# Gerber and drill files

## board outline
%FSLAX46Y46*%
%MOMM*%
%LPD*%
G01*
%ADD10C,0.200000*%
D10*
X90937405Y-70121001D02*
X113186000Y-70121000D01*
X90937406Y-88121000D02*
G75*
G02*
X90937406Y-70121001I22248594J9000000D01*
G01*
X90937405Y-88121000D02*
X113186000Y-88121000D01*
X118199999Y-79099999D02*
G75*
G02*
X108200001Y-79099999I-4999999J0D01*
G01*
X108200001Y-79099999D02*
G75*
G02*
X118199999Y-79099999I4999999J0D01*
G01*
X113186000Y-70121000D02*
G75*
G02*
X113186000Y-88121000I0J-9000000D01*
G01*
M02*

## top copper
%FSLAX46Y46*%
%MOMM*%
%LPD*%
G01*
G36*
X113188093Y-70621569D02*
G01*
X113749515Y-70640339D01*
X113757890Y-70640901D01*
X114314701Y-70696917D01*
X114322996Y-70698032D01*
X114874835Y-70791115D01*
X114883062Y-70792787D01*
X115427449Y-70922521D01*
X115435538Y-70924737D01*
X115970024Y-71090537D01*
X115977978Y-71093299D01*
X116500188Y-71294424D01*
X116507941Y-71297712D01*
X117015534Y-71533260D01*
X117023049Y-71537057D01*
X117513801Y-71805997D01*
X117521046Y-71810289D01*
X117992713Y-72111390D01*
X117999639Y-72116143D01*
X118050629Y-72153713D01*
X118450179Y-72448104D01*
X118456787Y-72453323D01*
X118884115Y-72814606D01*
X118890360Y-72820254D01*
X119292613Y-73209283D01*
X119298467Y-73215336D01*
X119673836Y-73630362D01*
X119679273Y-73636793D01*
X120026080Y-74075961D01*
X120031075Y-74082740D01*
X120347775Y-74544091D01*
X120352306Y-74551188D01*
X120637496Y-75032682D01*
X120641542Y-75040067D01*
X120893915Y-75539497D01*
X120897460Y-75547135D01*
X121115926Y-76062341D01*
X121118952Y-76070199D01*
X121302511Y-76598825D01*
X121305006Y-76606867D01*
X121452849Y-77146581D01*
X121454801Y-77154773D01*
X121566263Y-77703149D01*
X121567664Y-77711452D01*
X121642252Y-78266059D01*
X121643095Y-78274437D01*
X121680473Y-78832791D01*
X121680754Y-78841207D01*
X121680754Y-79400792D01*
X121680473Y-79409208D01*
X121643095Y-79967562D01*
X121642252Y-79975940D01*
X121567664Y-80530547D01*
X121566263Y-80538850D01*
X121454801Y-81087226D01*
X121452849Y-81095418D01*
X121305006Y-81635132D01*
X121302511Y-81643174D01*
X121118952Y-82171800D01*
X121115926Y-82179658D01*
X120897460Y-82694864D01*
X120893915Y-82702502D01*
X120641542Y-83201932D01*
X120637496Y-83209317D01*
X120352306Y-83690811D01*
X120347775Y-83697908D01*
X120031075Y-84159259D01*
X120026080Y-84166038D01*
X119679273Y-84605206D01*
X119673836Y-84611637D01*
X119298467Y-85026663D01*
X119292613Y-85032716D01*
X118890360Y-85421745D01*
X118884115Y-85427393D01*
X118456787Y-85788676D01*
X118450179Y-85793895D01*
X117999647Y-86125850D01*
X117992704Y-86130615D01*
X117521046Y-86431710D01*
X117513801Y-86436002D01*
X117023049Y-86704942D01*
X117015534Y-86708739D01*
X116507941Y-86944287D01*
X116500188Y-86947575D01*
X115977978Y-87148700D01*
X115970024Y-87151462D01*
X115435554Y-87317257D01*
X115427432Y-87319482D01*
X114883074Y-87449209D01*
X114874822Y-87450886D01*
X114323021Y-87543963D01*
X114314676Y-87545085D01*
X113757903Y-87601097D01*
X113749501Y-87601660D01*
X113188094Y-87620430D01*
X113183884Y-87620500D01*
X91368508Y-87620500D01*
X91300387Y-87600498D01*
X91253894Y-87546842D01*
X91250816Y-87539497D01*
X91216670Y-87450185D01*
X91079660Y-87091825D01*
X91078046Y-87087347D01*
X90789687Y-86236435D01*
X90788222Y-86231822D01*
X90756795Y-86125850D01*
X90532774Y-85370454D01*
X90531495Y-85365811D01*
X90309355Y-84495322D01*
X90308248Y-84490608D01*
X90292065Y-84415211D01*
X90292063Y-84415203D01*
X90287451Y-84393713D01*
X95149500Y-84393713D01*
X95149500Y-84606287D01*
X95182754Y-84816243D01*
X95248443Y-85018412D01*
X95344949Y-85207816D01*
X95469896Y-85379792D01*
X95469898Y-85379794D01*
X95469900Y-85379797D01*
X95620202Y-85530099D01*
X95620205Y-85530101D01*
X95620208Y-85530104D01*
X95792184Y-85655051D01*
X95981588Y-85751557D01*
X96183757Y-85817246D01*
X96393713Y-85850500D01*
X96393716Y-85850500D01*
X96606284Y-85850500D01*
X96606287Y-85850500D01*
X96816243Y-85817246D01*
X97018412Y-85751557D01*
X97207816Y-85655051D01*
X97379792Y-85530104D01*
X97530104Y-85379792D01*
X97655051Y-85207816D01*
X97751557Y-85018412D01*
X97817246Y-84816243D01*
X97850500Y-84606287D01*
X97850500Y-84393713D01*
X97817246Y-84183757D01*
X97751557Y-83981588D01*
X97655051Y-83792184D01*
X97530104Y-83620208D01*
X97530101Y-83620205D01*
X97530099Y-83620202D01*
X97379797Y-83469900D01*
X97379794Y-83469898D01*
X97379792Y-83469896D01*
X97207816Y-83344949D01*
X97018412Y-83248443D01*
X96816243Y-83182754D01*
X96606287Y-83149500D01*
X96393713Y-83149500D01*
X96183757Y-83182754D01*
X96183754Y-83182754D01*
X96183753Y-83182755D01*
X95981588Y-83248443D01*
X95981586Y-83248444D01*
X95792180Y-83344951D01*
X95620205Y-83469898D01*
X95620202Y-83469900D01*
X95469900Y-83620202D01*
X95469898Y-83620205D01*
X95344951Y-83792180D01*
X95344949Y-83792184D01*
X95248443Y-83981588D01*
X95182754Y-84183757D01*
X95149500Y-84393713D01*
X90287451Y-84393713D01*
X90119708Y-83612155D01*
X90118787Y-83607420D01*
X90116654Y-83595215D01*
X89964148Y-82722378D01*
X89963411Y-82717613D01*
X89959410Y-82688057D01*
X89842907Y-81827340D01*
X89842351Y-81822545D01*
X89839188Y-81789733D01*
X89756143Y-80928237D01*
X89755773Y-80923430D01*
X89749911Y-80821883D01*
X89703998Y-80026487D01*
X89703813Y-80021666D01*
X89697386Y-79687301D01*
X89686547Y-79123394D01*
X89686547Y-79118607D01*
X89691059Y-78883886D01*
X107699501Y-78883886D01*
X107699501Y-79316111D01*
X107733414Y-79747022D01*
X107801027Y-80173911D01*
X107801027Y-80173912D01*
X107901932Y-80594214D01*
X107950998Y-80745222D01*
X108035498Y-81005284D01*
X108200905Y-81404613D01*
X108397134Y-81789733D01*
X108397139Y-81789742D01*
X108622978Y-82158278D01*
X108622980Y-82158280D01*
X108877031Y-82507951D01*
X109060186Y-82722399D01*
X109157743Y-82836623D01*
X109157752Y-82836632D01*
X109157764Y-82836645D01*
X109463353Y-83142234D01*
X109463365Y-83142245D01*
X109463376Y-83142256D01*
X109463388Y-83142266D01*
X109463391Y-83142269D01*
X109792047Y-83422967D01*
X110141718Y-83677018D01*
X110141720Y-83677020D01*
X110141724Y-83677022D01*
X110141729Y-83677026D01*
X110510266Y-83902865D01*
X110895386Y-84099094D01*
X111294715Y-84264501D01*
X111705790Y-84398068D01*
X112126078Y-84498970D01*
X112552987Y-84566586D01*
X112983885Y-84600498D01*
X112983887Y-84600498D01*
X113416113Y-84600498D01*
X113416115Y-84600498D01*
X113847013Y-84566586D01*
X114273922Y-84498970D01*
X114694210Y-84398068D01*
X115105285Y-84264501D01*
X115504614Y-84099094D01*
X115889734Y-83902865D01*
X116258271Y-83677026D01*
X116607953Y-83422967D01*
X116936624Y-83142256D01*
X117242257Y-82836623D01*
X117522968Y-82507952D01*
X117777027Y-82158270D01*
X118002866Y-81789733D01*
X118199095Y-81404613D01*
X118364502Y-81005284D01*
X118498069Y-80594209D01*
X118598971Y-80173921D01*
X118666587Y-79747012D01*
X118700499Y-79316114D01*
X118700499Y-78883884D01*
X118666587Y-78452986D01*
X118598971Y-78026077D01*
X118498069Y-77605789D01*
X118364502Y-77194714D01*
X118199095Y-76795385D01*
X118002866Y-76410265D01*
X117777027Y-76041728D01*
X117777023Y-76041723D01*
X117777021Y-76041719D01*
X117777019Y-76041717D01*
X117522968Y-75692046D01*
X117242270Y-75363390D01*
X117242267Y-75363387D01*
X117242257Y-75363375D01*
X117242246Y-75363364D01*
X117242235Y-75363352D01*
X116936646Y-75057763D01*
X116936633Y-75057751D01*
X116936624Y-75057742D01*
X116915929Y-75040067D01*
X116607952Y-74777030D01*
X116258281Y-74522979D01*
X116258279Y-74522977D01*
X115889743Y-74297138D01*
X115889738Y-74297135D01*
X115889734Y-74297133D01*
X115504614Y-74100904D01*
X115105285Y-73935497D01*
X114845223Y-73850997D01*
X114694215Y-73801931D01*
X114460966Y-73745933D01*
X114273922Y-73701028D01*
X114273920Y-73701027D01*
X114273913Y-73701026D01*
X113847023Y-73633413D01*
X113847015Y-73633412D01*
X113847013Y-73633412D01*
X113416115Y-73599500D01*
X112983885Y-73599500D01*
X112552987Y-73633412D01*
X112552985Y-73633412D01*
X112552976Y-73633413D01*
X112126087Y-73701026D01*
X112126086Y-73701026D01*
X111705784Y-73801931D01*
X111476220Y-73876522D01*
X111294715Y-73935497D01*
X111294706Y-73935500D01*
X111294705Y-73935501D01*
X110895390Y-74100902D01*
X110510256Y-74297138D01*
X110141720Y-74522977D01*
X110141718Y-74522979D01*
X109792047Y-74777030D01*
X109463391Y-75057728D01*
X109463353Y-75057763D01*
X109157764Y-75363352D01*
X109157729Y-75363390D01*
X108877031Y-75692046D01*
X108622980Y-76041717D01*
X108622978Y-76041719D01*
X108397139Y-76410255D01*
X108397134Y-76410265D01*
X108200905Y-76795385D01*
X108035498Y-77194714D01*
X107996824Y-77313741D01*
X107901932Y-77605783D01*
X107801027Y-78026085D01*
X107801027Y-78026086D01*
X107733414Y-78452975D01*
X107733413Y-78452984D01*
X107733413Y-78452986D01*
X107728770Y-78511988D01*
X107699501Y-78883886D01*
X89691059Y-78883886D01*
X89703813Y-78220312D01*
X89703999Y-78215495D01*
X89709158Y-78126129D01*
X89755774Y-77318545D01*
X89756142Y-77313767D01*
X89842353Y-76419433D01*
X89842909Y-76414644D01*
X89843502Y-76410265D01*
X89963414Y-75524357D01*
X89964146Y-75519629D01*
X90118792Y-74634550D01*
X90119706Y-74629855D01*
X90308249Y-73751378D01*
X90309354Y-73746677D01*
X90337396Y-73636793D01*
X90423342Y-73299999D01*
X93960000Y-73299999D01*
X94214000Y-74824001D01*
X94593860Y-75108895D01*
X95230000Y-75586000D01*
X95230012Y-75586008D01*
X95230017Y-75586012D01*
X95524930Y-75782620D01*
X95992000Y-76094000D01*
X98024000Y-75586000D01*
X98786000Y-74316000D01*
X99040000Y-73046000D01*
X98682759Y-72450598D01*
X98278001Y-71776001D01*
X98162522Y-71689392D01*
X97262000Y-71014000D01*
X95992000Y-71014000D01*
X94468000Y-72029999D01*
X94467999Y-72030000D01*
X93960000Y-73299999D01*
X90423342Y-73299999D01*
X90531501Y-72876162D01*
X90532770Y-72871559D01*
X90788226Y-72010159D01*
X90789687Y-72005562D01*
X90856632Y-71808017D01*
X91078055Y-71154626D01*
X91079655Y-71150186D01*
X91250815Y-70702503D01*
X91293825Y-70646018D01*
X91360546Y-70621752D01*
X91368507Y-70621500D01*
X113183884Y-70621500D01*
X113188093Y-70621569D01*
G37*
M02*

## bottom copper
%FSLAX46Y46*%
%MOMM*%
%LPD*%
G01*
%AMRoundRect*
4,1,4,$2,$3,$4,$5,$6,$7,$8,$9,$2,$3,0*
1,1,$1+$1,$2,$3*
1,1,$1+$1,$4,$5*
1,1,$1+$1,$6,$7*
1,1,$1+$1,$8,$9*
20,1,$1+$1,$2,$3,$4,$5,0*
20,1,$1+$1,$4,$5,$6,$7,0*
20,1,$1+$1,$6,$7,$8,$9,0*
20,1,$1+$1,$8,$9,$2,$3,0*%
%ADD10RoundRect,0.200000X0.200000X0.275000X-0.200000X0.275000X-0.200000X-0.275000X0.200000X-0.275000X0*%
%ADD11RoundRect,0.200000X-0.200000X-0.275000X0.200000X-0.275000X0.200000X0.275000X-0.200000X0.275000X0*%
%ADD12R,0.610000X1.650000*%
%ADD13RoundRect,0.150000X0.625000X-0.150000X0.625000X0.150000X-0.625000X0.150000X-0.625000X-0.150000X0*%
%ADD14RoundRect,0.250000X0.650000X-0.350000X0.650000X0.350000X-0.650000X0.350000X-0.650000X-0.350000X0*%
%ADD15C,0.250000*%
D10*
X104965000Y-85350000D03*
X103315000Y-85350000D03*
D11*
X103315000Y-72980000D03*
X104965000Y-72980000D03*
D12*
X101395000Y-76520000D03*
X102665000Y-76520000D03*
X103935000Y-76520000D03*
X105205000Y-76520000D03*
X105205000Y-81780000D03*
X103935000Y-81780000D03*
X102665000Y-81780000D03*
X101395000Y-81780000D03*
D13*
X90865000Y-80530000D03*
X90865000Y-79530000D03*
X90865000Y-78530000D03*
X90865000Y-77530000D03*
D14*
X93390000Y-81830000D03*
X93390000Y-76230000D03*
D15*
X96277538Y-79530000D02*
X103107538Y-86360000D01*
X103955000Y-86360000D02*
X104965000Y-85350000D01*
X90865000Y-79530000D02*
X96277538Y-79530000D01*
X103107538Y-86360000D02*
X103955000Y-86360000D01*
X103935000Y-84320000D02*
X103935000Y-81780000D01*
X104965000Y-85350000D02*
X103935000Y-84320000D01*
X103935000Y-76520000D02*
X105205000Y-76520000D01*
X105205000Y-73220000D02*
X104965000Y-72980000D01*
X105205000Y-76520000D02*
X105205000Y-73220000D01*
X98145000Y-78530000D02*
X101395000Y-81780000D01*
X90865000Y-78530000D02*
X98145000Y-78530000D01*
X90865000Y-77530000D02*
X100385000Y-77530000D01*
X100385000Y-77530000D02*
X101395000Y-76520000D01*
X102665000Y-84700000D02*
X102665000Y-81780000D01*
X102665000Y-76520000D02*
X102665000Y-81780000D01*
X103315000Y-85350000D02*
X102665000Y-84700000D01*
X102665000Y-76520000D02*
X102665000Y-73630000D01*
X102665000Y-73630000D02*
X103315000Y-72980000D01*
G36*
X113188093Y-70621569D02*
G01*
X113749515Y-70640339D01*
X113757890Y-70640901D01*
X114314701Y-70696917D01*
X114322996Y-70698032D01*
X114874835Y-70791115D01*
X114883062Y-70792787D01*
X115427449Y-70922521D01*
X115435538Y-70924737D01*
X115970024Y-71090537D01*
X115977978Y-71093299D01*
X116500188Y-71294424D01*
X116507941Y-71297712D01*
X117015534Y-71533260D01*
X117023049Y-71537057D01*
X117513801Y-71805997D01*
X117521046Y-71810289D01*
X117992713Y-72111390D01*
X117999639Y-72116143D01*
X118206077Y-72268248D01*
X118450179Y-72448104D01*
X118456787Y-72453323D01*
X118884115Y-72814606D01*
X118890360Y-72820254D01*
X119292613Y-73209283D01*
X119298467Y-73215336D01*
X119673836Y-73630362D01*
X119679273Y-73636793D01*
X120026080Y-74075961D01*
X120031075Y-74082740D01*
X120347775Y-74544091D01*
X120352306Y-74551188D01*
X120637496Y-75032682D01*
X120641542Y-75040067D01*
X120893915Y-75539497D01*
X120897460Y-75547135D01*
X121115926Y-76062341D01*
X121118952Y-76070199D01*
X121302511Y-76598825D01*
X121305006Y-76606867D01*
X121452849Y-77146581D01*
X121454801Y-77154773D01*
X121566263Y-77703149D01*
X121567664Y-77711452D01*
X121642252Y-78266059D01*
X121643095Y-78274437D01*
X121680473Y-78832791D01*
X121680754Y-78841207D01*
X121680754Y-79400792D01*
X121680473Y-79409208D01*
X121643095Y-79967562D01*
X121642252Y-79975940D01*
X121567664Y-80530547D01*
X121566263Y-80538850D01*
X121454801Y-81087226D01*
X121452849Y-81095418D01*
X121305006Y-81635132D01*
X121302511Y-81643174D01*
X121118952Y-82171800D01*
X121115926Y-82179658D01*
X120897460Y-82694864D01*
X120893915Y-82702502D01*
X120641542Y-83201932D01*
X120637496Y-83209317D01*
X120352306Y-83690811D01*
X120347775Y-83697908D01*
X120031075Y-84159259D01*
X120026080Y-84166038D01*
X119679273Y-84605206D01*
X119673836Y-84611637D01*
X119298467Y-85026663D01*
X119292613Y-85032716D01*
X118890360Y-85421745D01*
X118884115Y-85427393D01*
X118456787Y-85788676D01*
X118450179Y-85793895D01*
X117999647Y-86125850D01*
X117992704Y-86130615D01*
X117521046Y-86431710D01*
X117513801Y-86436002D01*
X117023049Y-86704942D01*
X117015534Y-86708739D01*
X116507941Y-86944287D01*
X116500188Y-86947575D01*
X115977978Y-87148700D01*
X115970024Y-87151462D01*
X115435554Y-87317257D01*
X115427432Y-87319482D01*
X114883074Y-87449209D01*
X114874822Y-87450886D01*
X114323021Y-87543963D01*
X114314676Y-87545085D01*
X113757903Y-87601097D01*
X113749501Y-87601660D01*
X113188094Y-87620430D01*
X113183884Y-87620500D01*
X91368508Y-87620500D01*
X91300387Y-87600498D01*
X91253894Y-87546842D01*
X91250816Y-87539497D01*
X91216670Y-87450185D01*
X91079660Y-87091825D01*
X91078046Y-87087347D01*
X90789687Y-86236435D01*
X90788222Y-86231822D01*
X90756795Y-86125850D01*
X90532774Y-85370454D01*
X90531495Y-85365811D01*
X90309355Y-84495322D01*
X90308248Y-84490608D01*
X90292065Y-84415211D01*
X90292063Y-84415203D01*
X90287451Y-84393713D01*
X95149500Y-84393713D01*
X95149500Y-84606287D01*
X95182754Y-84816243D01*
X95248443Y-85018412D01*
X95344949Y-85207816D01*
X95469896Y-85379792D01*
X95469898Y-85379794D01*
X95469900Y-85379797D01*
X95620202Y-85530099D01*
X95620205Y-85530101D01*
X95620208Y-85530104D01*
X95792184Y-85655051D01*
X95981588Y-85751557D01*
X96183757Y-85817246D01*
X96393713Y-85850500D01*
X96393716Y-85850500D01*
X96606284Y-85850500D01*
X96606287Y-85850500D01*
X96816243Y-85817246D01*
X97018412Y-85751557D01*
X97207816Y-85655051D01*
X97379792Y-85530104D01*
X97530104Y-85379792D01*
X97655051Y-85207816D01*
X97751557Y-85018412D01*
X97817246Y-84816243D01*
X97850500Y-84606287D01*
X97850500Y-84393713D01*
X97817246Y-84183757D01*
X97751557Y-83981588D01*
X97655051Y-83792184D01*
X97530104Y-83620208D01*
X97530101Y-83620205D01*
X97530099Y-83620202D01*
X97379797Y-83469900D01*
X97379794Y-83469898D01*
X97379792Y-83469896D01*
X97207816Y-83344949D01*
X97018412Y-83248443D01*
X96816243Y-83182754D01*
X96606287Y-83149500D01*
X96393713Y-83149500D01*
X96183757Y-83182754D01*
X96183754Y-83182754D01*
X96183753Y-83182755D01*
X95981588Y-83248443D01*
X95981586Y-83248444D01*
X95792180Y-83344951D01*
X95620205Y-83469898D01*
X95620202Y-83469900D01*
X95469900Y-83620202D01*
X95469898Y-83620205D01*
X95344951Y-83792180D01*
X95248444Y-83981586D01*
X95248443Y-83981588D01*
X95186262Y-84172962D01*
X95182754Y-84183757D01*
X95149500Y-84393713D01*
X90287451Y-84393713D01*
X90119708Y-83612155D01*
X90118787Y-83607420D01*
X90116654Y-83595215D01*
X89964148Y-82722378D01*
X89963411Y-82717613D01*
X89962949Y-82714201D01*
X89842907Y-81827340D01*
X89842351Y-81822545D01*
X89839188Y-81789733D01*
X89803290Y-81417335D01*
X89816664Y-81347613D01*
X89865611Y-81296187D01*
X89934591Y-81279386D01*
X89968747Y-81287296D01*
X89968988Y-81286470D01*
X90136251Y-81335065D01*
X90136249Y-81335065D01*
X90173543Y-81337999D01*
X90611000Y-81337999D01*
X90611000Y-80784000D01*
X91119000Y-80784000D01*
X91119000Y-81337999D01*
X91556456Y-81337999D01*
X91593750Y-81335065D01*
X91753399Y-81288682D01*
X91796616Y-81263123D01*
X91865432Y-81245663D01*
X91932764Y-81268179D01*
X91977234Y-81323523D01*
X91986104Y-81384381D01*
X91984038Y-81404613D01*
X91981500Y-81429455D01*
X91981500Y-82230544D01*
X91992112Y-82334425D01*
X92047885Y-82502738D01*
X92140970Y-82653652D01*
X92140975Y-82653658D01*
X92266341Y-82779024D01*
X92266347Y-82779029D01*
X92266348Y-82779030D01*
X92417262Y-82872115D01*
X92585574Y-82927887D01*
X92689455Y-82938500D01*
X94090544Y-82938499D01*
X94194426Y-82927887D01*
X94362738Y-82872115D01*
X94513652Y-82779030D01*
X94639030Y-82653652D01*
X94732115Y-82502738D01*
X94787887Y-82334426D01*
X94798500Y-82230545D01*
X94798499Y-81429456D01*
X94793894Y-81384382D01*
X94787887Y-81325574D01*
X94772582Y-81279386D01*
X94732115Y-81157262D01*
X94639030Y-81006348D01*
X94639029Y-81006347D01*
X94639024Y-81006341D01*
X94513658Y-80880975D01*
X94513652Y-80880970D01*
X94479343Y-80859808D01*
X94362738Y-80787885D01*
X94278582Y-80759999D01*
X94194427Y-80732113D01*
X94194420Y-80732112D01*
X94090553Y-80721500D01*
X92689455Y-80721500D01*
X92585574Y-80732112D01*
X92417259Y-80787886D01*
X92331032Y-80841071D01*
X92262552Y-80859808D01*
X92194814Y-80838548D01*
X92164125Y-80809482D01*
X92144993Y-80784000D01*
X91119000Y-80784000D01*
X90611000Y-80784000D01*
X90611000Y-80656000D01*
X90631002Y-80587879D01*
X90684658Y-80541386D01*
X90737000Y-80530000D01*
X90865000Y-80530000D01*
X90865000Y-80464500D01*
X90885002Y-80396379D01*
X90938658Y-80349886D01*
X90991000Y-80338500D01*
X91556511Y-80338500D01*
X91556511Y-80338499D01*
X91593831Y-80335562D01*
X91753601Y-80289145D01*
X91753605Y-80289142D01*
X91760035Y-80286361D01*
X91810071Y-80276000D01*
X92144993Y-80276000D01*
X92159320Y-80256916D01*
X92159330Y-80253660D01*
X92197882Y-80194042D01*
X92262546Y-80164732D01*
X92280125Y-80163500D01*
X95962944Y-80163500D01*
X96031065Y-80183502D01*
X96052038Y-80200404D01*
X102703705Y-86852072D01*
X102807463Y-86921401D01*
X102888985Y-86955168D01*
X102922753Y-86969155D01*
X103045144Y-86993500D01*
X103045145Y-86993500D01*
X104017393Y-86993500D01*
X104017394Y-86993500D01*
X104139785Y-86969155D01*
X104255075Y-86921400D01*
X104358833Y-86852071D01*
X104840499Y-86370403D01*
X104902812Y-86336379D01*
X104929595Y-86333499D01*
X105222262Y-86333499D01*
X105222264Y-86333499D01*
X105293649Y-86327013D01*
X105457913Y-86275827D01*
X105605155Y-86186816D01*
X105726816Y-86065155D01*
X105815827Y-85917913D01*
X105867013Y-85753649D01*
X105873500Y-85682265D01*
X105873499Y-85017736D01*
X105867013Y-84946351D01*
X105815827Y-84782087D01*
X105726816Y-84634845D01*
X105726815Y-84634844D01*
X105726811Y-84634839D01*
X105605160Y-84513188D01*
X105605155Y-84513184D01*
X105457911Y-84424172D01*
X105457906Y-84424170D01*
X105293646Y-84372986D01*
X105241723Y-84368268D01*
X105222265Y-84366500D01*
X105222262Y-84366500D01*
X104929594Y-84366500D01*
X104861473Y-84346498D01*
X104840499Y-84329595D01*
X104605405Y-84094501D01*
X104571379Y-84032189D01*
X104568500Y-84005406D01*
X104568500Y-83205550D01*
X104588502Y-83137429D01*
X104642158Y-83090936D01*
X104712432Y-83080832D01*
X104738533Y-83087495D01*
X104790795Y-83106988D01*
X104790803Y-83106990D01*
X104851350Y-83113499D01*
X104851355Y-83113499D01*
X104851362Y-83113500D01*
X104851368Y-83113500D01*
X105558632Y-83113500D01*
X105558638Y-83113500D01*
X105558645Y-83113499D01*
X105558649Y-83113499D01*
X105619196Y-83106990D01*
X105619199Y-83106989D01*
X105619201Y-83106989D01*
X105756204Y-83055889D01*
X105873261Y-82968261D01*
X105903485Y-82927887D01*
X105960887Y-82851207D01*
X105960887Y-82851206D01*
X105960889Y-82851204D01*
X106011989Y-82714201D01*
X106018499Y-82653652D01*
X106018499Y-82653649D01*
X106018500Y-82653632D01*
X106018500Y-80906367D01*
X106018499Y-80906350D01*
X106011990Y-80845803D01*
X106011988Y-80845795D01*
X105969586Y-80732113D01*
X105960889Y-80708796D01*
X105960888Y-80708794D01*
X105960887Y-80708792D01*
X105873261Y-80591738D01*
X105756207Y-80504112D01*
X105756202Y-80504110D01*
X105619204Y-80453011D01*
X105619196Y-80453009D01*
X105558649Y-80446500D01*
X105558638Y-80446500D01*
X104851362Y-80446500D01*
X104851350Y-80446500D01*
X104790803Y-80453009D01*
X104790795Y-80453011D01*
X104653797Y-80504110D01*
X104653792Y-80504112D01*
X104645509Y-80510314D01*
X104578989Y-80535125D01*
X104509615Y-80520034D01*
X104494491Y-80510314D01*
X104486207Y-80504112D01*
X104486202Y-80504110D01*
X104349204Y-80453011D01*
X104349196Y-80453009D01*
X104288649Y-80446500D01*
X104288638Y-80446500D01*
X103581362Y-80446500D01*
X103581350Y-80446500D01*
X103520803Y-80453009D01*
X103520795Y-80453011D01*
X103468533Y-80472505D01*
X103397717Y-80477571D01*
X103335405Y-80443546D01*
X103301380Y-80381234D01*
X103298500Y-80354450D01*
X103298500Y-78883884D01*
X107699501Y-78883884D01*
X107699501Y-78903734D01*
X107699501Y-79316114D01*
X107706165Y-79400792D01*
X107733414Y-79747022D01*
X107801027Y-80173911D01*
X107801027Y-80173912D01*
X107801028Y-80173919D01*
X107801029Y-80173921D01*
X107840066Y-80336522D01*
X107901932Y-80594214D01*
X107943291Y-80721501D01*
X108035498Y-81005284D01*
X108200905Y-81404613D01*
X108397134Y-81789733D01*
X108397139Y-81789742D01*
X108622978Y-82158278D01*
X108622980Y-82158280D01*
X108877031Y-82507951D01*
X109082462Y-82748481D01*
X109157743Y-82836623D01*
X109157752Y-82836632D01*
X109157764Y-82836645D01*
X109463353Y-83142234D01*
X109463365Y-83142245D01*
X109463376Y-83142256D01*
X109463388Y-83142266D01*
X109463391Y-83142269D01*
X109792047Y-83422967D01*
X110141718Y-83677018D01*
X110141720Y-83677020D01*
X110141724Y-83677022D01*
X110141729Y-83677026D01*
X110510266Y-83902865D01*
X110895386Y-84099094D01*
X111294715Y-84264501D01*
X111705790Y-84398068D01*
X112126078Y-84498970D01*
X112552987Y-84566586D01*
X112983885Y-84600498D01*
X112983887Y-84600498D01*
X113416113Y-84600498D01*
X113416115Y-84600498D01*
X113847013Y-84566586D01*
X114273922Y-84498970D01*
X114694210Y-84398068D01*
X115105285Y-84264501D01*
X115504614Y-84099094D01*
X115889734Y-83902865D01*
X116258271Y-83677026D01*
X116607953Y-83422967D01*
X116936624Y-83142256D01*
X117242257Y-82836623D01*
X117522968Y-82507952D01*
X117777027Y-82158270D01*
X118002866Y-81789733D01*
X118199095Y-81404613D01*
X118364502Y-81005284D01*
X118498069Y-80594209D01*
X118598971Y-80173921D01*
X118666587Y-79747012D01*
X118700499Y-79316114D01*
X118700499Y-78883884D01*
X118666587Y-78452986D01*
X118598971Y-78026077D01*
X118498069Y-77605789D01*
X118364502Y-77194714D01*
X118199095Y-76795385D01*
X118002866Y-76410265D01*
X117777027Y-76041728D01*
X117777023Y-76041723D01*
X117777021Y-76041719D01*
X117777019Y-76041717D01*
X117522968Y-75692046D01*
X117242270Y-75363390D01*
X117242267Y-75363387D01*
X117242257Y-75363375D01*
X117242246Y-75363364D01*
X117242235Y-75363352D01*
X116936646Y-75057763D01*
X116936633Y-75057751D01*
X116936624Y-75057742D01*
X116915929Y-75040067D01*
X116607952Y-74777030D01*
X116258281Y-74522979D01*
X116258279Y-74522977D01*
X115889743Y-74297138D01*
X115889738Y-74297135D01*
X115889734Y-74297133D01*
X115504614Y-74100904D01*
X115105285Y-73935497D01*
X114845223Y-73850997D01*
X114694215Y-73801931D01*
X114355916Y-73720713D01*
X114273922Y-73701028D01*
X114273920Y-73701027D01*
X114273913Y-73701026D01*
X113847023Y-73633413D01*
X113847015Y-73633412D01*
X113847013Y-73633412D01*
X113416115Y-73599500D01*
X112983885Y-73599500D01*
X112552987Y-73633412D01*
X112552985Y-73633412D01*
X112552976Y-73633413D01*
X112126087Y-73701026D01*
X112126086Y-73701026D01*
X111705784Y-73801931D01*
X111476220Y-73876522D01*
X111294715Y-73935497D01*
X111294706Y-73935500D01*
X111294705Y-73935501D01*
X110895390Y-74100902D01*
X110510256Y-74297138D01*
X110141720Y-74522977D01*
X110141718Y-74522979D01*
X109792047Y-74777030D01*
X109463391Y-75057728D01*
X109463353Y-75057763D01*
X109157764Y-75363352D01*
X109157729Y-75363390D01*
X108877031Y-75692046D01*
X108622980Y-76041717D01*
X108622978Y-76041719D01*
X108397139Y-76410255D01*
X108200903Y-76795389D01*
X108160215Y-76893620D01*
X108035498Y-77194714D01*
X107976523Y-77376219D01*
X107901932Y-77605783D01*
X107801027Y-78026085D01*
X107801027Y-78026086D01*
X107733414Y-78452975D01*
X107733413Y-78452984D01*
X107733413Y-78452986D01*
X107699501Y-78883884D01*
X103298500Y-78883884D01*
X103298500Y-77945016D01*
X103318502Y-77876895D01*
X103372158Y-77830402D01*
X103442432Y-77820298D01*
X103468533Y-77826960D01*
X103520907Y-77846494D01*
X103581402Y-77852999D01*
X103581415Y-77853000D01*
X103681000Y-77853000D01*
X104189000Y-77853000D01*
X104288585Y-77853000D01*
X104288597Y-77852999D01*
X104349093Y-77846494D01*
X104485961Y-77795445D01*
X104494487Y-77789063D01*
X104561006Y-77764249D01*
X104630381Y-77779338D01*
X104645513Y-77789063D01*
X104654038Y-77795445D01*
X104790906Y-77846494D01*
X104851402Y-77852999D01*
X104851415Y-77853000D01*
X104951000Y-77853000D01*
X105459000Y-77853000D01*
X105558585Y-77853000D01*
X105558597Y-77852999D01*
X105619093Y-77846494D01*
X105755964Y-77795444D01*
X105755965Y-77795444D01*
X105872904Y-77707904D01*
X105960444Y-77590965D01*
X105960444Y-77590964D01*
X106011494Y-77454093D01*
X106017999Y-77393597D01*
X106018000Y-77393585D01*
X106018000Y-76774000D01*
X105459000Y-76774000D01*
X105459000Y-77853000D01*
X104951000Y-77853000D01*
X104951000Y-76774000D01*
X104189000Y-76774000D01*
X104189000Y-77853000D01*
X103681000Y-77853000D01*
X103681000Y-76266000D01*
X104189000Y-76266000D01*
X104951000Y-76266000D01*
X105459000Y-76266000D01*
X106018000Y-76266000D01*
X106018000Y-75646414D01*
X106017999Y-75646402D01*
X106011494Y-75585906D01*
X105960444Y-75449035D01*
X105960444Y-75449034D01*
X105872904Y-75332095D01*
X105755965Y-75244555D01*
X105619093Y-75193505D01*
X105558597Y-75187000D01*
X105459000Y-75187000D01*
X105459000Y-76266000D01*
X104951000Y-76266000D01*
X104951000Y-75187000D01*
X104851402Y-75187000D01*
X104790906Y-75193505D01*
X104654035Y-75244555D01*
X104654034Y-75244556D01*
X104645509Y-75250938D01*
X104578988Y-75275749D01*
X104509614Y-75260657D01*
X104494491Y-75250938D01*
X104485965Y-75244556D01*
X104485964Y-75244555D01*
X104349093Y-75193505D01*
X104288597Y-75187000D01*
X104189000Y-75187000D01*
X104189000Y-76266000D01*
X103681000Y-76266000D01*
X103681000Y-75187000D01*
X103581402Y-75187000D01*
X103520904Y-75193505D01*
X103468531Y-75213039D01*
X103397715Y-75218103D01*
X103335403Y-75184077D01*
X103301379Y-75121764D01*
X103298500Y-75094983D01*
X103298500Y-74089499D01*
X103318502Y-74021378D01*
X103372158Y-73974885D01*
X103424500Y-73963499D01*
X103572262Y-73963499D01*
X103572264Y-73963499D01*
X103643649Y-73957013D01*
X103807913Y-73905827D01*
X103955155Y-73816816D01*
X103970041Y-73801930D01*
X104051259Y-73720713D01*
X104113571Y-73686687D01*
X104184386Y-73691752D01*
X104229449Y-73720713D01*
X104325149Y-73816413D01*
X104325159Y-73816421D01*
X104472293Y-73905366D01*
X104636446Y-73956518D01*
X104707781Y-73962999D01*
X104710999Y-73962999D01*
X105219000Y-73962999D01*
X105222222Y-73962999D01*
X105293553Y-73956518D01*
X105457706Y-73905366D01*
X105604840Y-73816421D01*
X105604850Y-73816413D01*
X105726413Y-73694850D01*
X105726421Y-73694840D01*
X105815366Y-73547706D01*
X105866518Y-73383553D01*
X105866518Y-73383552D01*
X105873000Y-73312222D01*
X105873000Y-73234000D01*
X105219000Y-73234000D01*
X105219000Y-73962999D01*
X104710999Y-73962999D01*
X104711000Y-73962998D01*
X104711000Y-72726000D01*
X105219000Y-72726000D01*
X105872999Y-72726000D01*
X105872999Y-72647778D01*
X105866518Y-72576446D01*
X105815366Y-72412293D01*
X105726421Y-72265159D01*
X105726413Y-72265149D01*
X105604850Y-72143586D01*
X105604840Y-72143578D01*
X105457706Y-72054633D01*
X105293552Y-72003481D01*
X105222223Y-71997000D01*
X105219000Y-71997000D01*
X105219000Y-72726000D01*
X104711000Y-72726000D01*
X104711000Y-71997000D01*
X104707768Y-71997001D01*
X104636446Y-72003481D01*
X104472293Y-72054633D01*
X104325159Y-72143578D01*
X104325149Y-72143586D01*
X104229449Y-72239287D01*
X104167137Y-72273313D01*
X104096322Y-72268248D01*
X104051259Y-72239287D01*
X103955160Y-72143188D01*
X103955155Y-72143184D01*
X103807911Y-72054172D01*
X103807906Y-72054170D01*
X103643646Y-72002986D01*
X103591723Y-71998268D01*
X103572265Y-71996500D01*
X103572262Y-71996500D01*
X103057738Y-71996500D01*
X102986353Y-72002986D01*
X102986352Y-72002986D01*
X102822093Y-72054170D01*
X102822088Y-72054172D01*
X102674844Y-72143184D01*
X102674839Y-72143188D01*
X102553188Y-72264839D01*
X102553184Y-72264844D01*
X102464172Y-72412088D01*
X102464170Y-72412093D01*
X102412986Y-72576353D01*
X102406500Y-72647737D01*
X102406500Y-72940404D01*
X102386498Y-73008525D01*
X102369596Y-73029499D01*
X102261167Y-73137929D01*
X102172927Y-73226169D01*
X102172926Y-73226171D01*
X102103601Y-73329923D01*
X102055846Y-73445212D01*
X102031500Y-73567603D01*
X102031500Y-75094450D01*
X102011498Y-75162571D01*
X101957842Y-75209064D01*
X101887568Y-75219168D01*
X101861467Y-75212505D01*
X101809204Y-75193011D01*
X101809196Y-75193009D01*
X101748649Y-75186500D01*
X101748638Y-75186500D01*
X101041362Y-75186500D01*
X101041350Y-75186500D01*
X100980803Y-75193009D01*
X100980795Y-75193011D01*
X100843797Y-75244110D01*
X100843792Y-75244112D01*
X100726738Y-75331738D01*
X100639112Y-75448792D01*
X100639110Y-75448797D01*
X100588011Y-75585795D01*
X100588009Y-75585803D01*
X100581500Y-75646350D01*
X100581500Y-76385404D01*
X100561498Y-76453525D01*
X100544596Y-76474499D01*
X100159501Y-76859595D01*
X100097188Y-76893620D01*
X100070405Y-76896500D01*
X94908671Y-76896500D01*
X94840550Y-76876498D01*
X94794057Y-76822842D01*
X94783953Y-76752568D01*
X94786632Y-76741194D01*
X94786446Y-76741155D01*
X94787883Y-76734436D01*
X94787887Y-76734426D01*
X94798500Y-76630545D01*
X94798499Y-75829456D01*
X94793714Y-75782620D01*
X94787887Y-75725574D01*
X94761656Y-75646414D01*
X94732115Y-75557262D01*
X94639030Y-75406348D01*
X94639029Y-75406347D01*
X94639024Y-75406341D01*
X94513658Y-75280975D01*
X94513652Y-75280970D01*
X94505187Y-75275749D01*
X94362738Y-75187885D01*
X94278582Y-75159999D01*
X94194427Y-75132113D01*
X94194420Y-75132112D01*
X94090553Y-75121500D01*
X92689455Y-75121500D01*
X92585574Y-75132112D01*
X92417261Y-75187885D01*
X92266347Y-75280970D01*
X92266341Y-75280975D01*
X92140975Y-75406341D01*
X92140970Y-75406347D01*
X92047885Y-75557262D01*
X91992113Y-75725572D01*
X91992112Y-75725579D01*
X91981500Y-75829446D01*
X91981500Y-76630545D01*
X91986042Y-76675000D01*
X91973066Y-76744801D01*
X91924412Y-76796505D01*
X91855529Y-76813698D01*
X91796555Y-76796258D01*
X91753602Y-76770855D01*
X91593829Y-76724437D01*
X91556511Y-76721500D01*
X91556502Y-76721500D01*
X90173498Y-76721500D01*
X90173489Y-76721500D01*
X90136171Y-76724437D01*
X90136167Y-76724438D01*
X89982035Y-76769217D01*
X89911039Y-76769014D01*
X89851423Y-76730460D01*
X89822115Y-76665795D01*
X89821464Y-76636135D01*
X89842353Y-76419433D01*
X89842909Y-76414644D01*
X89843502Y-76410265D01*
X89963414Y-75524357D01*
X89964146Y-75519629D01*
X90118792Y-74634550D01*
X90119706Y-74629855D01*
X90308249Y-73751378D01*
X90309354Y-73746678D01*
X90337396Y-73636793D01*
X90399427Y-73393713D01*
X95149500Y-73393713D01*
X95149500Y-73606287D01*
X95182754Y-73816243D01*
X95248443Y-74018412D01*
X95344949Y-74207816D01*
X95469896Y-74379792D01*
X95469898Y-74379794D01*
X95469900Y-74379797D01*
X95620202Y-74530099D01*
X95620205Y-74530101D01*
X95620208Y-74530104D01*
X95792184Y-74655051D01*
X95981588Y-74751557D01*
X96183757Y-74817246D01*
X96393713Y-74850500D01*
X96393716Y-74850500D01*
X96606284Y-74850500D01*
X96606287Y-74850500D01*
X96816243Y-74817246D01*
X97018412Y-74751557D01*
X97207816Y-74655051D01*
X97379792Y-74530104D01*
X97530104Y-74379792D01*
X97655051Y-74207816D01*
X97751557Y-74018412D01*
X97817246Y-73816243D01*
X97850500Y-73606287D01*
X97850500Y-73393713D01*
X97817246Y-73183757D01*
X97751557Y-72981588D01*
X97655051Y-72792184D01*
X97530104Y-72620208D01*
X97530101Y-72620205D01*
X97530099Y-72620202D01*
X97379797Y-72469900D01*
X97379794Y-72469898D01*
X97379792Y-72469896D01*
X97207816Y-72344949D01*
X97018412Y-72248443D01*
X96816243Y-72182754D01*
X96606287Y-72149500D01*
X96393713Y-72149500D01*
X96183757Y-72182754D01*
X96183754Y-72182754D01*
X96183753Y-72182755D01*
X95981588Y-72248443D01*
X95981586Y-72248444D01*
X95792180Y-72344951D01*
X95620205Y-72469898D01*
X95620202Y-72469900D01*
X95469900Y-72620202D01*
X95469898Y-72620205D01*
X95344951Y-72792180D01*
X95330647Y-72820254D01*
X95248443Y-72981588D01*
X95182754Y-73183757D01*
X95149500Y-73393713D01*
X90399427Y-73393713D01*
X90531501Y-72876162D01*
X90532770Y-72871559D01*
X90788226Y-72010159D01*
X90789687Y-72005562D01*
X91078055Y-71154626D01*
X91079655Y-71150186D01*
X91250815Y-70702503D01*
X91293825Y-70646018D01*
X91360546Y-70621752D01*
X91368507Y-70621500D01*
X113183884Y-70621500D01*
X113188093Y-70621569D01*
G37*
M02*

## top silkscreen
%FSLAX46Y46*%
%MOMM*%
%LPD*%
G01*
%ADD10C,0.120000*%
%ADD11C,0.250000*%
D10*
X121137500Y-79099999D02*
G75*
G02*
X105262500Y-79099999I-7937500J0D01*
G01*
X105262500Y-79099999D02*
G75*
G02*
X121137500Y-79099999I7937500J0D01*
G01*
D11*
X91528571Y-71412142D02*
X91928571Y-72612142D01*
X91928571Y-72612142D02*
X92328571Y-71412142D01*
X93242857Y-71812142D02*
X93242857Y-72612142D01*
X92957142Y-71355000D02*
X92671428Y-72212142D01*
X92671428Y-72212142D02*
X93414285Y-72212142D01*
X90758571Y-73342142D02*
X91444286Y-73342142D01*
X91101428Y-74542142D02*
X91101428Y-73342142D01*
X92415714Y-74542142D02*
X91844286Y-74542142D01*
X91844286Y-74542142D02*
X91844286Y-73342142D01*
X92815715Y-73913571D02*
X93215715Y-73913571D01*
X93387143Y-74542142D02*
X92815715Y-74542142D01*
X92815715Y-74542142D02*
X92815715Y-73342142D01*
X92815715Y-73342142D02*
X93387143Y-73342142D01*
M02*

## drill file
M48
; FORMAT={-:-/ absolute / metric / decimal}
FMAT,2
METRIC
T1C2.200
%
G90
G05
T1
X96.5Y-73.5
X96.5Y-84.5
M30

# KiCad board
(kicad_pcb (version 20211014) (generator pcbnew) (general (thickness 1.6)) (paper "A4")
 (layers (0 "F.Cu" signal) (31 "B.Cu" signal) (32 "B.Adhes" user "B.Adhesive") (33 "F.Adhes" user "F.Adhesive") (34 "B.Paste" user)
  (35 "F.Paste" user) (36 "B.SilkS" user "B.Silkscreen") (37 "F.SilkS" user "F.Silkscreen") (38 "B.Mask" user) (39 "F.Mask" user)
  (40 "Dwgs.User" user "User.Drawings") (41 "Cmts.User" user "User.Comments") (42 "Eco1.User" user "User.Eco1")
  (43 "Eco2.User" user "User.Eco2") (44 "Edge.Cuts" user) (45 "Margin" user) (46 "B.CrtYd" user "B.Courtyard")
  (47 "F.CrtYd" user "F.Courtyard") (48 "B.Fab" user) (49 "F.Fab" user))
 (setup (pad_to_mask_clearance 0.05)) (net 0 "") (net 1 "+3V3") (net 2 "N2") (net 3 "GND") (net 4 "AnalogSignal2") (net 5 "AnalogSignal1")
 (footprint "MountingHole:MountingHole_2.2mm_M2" (layer "F.Cu") (at 96.5 84.5)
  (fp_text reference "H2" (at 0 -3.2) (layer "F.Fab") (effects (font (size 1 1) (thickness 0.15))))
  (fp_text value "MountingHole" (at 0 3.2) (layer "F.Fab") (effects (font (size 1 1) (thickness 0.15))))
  (pad "" np_thru_hole circle locked (at 0 0) (size 2.2 2.2) (drill 2.2) (layers *.Cu *.Mask)))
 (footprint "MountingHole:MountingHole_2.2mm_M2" (layer "F.Cu") (at 96.5 73.5)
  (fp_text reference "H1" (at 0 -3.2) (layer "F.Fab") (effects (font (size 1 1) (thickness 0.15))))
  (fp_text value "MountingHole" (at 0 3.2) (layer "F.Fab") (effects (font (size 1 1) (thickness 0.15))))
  (pad "" np_thru_hole circle locked (at 0 0) (size 2.2 2.2) (drill 2.2) (layers *.Cu *.Mask)))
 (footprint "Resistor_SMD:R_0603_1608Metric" (layer "B.Cu") (at 104.14 85.35 180)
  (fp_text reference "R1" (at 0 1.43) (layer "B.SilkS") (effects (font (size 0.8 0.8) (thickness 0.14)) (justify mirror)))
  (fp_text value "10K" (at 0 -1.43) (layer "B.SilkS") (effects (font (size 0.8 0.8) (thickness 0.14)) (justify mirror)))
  (pad "1" smd roundrect locked (at -0.825 0 180) (size 0.8 0.95) (layers "B.Cu" "B.Paste" "B.Mask") (roundrect_rratio 0.25) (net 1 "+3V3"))
  (pad "2" smd roundrect locked (at 0.825 0 180) (size 0.8 0.95) (layers "B.Cu" "B.Paste" "B.Mask") (roundrect_rratio 0.25) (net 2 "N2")))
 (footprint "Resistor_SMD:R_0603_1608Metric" (layer "B.Cu") (at 104.14 72.98)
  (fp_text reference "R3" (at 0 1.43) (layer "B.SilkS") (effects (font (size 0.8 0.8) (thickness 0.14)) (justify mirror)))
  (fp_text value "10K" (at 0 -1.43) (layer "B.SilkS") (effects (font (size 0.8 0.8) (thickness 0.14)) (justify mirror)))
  (pad "1" smd roundrect locked (at -0.825 0) (size 0.8 0.95) (layers "B.Cu" "B.Paste" "B.Mask") (roundrect_rratio 0.25) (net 2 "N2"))
  (pad "2" smd roundrect locked (at 0.825 0) (size 0.8 0.95) (layers "B.Cu" "B.Paste" "B.Mask") (roundrect_rratio 0.25) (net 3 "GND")))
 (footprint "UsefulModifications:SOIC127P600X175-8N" (layer "B.Cu") (at 103.3 79.15 -90)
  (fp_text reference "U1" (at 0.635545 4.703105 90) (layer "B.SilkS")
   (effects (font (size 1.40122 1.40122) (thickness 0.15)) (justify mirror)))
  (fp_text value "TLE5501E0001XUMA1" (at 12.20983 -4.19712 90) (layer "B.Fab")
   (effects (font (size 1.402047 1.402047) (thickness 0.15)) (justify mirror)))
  (pad "1" smd rect locked (at -2.63 1.905 270) (size 1.65 0.61) (layers "B.Cu" "B.Paste" "B.Mask") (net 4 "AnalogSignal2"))
  (pad "2" smd rect locked (at -2.63 0.635 270) (size 1.65 0.61) (layers "B.Cu" "B.Paste" "B.Mask") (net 2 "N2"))
  (pad "3" smd rect locked (at -2.63 -0.635 270) (size 1.65 0.61) (layers "B.Cu" "B.Paste" "B.Mask") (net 3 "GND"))
  (pad "4" smd rect locked (at -2.63 -1.905 270) (size 1.65 0.61) (layers "B.Cu" "B.Paste" "B.Mask") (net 3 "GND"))
  (pad "5" smd rect locked (at 2.63 -1.905 270) (size 1.65 0.61) (layers "B.Cu" "B.Paste" "B.Mask"))
  (pad "6" smd rect locked (at 2.63 -0.635 270) (size 1.65 0.61) (layers "B.Cu" "B.Paste" "B.Mask") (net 1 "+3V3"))
  (pad "7" smd rect locked (at 2.63 0.635 270) (size 1.65 0.61) (layers "B.Cu" "B.Paste" "B.Mask") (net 2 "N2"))
  (pad "8" smd rect locked (at 2.63 1.905 270) (size 1.65 0.61) (layers "B.Cu" "B.Paste" "B.Mask") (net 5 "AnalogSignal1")))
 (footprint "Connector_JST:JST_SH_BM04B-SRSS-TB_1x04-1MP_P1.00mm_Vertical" (layer "B.Cu") (at 92.19 79.03 90)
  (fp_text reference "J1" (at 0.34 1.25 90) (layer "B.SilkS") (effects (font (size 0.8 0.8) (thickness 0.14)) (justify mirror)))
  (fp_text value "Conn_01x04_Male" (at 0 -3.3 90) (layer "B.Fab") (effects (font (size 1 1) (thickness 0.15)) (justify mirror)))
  (pad "1" smd roundrect locked (at -1.5 -1.325 90) (size 0.6 1.55) (layers "B.Cu" "B.Paste" "B.Mask") (roundrect_rratio 0.25) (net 3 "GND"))
  (pad "2" smd roundrect locked (at -0.5 -1.325 90) (size 0.6 1.55) (layers "B.Cu" "B.Paste" "B.Mask") (roundrect_rratio 0.25)
   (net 1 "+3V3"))
  (pad "3" smd roundrect locked (at 0.5 -1.325 90) (size 0.6 1.55) (layers "B.Cu" "B.Paste" "B.Mask") (roundrect_rratio 0.25)
   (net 5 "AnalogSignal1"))
  (pad "4" smd roundrect locked (at 1.5 -1.325 90) (size 0.6 1.55) (layers "B.Cu" "B.Paste" "B.Mask") (roundrect_rratio 0.25)
   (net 4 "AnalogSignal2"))
  (pad "MP" smd roundrect locked (at -2.8 1.2 90) (size 1.2 1.8) (layers "B.Cu" "B.Paste" "B.Mask") (roundrect_rratio 0.2083333333))
  (pad "MP" smd roundrect locked (at 2.8 1.2 90) (size 1.2 1.8) (layers "B.Cu" "B.Paste" "B.Mask") (roundrect_rratio 0.2083333333)))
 (gr_circle (center 113.2 79.099999) (end 121.1375 79.099999) (layer "F.SilkS") (width 0.12) (fill none))
 (gr_line (start 90.937405 70.121001) (end 113.186 70.121) (layer "Edge.Cuts") (width 0.2))
 (gr_arc (start 90.937406 88.121) (mid 89.186001 79.121001) (end 90.937405 70.121001) (layer "Edge.Cuts") (width 0.2))
 (gr_line (start 90.937405 88.121) (end 113.186 88.121) (layer "Edge.Cuts") (width 0.2))
 (gr_circle (center 113.2 79.099999) (end 118.199999 79.099999) (layer "Edge.Cuts") (width 0.2) (fill none))
 (gr_arc (start 113.186 70.121) (mid 122.186 79.121) (end 113.186 88.121) (layer "Edge.Cuts") (width 0.2))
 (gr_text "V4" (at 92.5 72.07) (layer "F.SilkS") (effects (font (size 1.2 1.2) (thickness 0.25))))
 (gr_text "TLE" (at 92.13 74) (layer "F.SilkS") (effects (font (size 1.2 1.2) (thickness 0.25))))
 (segment (start 96.277538 79.53) (end 103.107538 86.36) (width 0.25) (layer "B.Cu") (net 1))
 (segment (start 103.955 86.36) (end 104.965 85.35) (width 0.25) (layer "B.Cu") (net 1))
 (segment (start 90.865 79.53) (end 96.277538 79.53) (width 0.25) (layer "B.Cu") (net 1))
 (segment (start 103.107538 86.36) (end 103.955 86.36) (width 0.25) (layer "B.Cu") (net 1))
 (segment (start 103.935 84.32) (end 103.935 81.78) (width 0.25) (layer "B.Cu") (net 1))
 (segment (start 104.965 85.35) (end 103.935 84.32) (width 0.25) (layer "B.Cu") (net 1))
 (segment (start 103.935 76.52) (end 105.205 76.52) (width 0.25) (layer "B.Cu") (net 3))
 (segment (start 105.205 73.22) (end 104.965 72.98) (width 0.25) (layer "B.Cu") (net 3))
 (segment (start 105.205 76.52) (end 105.205 73.22) (width 0.25) (layer "B.Cu") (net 3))
 (segment (start 98.145 78.53) (end 101.395 81.78) (width 0.25) (layer "B.Cu") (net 5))
 (segment (start 90.865 78.53) (end 98.145 78.53) (width 0.25) (layer "B.Cu") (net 5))
 (segment (start 90.865 77.53) (end 100.385 77.53) (width 0.25) (layer "B.Cu") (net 4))
 (segment (start 100.385 77.53) (end 101.395 76.52) (width 0.25) (layer "B.Cu") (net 4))
 (segment (start 102.665 84.7) (end 102.665 81.78) (width 0.25) (layer "B.Cu") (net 2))
 (segment (start 102.665 76.52) (end 102.665 81.78) (width 0.25) (layer "B.Cu") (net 2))
 (segment (start 103.315 85.35) (end 102.665 84.7) (width 0.25) (layer "B.Cu") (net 2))
 (segment (start 102.665 76.52) (end 102.665 73.63) (width 0.25) (layer "B.Cu") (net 2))
 (segment (start 102.665 73.63) (end 103.315 72.98) (width 0.25) (layer "B.Cu") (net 2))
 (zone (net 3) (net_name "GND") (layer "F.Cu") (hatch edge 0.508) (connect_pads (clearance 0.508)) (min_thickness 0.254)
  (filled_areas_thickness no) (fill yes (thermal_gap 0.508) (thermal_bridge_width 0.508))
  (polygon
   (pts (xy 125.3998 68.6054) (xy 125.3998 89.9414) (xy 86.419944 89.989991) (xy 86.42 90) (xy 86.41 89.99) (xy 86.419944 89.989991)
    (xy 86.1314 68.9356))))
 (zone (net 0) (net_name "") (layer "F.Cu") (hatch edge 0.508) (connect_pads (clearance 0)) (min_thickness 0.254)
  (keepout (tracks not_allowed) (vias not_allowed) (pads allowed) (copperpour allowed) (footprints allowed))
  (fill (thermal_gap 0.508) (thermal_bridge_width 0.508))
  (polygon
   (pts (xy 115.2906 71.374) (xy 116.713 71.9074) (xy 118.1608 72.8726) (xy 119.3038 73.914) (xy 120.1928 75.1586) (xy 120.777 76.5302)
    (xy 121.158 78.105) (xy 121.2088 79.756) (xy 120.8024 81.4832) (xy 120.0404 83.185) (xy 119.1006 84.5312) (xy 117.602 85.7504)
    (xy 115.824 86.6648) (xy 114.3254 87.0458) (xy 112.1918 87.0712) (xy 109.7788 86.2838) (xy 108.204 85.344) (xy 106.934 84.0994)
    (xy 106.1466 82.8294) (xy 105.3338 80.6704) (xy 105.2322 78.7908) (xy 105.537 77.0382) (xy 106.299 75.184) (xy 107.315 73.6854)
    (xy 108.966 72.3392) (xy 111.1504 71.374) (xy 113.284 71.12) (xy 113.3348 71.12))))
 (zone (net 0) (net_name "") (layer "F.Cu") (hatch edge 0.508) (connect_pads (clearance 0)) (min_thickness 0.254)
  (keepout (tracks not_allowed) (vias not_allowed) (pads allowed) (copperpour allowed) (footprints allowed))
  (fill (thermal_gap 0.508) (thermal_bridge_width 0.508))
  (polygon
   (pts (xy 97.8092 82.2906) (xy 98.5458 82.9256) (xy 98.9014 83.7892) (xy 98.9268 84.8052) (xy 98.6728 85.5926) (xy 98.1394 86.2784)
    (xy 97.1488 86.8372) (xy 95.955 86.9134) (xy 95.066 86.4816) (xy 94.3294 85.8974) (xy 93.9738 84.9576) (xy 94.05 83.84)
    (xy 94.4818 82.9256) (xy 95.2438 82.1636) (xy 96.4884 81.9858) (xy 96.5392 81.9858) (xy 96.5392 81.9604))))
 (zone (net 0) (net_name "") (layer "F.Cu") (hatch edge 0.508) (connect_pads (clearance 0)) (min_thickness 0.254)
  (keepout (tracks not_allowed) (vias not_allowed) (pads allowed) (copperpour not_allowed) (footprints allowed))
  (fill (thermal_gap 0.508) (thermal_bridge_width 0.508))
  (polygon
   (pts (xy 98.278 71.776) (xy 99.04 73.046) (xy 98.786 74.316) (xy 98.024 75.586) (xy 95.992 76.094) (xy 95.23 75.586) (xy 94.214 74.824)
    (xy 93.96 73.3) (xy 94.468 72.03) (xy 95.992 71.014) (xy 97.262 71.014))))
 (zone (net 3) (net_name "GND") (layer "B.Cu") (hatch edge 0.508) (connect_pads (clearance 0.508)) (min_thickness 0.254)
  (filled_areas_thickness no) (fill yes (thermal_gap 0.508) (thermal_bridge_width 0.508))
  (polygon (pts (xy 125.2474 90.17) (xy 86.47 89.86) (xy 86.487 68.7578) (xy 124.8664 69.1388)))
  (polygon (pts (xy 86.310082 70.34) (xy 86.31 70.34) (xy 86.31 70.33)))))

